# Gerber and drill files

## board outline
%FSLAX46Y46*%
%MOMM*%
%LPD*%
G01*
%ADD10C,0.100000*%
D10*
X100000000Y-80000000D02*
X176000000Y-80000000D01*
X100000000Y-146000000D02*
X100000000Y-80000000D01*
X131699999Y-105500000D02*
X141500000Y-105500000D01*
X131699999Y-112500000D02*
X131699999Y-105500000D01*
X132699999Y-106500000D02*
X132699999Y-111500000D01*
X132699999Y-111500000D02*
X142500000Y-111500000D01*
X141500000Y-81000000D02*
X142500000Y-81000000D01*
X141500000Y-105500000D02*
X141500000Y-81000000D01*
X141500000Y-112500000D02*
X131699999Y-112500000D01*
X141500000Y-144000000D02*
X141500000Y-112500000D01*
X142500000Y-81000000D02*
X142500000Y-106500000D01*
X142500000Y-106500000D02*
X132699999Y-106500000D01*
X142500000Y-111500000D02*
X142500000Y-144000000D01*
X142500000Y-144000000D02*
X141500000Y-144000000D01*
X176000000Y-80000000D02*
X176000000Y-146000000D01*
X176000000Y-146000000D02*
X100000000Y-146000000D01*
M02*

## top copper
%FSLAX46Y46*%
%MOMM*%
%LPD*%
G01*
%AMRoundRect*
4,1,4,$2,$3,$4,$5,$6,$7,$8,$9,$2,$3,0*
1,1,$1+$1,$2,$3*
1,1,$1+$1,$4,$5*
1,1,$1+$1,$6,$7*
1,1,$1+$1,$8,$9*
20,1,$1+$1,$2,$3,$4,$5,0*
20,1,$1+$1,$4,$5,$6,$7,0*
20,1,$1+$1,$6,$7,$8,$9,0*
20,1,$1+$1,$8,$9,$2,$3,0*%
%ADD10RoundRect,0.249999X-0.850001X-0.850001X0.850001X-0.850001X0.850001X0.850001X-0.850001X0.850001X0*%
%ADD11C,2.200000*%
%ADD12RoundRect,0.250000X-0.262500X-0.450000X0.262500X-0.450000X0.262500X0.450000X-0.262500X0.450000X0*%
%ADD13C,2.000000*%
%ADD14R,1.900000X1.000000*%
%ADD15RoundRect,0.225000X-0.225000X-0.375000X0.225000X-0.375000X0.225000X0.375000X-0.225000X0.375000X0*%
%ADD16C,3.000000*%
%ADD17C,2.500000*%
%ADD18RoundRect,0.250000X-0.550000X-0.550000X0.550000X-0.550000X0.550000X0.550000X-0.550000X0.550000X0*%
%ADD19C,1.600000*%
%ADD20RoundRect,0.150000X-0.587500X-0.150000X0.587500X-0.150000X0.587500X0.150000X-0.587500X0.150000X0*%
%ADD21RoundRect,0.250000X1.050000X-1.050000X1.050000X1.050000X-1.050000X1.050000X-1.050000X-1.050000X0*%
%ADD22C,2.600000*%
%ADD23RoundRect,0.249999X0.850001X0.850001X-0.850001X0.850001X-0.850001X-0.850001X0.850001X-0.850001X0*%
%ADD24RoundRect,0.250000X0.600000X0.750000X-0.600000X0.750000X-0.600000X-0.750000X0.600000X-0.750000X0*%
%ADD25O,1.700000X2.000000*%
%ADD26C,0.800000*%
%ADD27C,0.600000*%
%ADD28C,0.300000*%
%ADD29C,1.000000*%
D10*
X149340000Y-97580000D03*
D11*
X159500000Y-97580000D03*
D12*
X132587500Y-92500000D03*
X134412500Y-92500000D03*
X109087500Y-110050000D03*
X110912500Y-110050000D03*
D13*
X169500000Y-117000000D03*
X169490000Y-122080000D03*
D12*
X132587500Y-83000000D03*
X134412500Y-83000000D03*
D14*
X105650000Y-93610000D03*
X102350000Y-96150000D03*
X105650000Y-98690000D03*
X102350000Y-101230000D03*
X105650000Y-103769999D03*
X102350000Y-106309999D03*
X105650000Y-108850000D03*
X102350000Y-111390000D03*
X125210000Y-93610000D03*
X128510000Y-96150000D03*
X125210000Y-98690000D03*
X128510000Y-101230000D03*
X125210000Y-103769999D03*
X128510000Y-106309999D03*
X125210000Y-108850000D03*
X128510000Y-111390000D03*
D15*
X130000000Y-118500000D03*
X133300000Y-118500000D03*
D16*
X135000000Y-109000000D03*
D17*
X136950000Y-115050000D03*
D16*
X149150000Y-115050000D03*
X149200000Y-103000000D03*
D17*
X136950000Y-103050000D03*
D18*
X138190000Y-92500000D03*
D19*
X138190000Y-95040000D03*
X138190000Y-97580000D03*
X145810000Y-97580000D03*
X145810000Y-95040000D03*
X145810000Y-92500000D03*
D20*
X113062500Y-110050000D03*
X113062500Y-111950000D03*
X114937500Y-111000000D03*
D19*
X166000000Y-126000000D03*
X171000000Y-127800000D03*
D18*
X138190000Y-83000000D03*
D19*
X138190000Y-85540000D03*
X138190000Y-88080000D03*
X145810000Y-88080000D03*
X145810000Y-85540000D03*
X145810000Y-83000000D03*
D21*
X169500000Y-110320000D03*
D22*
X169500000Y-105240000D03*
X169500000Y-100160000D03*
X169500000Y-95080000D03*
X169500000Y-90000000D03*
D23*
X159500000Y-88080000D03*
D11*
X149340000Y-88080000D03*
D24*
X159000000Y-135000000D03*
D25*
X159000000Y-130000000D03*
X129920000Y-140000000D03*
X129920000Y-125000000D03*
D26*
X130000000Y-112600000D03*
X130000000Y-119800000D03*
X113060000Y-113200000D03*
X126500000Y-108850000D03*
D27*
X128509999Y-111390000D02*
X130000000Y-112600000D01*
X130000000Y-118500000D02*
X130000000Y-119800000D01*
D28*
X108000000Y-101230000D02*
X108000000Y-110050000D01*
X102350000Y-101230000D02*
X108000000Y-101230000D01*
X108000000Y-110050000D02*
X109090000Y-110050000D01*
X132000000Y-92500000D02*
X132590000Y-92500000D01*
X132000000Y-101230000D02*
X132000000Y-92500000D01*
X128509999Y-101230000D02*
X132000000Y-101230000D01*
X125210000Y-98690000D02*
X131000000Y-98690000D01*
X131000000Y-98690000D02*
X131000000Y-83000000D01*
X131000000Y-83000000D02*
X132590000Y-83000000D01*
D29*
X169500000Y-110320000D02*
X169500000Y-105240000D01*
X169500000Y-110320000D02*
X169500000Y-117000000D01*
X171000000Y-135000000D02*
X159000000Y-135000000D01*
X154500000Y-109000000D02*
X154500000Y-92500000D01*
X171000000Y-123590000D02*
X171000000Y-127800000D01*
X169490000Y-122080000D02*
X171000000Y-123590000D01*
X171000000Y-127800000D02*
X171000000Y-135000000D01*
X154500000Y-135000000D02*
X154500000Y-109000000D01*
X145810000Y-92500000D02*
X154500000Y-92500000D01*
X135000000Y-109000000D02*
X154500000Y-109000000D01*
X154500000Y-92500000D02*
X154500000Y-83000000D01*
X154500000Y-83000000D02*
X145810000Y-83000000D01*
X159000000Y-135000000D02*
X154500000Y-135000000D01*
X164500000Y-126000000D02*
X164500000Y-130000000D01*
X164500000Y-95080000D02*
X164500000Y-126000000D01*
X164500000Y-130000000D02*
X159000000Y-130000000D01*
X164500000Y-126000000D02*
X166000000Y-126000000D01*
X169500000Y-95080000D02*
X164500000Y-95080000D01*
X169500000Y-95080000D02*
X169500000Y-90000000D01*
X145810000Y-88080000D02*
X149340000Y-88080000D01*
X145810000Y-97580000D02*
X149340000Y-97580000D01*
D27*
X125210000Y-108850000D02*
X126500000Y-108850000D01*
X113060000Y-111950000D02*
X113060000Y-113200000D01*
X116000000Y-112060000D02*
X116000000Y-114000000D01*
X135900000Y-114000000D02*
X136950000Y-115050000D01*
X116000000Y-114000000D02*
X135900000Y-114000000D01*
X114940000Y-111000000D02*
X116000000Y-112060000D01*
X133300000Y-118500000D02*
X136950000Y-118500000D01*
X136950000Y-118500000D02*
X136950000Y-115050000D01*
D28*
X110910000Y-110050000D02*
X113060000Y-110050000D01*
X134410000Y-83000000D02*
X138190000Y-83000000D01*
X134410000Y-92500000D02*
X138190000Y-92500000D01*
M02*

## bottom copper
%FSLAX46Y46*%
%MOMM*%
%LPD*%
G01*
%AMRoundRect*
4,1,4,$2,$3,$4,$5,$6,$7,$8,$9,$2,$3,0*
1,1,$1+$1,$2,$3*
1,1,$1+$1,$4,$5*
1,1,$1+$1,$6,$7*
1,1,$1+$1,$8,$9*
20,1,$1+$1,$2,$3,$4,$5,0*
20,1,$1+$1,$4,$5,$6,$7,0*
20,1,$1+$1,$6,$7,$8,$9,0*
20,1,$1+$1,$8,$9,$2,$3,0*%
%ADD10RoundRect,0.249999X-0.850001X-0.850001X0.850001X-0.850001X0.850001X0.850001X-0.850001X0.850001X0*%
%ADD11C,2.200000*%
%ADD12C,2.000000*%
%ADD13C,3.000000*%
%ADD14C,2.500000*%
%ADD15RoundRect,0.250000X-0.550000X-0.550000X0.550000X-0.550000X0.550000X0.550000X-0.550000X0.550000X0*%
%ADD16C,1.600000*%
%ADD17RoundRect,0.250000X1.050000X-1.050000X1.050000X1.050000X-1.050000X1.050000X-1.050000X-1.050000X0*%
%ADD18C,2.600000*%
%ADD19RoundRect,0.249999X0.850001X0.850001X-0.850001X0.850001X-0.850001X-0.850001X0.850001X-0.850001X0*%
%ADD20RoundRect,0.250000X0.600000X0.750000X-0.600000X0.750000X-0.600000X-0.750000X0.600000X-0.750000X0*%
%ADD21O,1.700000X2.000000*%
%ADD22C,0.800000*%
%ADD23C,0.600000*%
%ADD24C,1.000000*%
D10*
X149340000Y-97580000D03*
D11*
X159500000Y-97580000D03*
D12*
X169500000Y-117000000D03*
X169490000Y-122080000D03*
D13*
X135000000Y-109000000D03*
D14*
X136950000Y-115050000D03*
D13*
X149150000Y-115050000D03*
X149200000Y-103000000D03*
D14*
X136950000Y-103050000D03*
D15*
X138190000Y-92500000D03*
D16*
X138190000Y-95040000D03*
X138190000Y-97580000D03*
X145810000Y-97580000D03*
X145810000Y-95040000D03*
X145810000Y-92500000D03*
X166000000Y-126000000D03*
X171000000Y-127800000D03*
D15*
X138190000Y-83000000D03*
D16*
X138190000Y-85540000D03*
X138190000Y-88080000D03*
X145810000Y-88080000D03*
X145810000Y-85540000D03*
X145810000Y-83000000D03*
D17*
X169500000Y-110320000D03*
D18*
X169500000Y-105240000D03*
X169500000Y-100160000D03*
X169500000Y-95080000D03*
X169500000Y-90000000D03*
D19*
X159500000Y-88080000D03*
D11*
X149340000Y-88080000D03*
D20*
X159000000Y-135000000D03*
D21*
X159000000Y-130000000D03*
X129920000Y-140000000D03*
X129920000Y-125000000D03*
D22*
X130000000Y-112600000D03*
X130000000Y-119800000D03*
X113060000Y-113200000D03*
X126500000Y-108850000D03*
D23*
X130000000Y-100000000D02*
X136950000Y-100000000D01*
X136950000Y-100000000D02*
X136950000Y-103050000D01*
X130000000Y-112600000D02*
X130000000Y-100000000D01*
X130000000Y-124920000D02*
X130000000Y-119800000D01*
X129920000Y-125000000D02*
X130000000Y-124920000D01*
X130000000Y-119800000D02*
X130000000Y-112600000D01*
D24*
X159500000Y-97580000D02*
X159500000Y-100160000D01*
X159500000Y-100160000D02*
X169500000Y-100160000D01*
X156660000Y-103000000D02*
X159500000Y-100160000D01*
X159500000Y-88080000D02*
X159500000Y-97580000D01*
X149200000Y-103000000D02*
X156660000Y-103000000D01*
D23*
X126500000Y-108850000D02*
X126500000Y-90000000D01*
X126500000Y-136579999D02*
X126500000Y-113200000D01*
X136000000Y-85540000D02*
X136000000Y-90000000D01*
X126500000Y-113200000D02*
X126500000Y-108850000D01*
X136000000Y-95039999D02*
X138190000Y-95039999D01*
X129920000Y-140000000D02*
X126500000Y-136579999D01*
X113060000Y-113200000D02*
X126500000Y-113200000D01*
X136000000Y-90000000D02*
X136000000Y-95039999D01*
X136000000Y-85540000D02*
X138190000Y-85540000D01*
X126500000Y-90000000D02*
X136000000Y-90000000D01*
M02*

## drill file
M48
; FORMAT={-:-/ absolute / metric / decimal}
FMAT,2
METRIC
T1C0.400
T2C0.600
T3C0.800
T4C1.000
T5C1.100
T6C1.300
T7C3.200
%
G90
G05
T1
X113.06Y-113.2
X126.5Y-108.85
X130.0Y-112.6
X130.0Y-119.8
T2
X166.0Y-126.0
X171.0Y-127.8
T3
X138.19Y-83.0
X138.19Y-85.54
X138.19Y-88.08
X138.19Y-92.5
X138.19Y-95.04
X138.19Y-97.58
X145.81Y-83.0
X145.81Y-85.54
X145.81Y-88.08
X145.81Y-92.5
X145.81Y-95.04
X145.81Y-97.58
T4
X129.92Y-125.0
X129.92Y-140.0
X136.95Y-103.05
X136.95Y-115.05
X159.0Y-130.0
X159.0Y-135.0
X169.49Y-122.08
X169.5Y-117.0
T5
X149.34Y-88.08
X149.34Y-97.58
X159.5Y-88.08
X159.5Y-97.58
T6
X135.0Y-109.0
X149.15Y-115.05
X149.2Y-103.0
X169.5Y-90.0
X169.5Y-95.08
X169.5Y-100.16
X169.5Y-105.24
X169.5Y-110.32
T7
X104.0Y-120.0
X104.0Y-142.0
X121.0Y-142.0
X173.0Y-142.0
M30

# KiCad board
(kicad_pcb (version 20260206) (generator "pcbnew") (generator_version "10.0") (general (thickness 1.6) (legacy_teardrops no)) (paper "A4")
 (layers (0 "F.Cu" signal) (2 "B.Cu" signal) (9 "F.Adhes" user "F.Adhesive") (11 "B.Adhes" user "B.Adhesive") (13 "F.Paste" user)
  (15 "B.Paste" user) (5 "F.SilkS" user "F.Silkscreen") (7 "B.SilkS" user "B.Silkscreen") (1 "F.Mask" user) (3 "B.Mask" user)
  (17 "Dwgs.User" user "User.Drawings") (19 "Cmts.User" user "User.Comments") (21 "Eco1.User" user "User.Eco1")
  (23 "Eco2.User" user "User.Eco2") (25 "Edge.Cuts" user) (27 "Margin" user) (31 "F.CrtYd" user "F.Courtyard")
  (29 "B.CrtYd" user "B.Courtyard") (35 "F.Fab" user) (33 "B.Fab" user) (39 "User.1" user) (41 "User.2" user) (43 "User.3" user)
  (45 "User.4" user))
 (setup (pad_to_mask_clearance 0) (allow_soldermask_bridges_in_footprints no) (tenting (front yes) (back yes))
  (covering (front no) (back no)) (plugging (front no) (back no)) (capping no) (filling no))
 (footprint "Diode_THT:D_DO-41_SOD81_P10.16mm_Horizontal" (layer "F.Cu") (at 149.34 97.58)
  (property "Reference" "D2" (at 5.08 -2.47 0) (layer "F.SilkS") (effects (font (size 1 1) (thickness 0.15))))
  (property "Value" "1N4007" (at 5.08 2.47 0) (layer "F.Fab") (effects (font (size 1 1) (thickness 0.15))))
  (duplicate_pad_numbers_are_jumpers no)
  (pad "1" thru_hole roundrect (at 0 0) (size 2.2 2.2) (drill 1.1) (layers "*.Cu" "*.Mask") (remove_unused_layers no)
   (roundrect_rratio 0.113636) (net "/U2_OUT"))
  (pad "2" thru_hole circle (at 10.16 0) (size 2.2 2.2) (drill 1.1) (layers "*.Cu" "*.Mask") (remove_unused_layers no) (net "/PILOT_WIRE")))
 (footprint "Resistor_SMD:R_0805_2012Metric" (layer "F.Cu") (at 133.5 92.5)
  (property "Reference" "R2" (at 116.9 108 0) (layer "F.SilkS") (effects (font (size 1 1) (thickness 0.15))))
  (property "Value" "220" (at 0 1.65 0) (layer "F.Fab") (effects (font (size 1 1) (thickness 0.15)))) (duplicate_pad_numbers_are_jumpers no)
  (pad "1" smd roundrect (at -0.9125 0) (size 1.025 1.4) (layers "F.Cu" "F.Mask" "F.Paste") (roundrect_rratio 0.243902) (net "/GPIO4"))
  (pad "2" smd roundrect (at 0.9125 0) (size 1.025 1.4) (layers "F.Cu" "F.Mask" "F.Paste") (roundrect_rratio 0.243902) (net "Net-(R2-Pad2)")))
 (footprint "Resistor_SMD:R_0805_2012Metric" (layer "F.Cu") (at 110 110.05)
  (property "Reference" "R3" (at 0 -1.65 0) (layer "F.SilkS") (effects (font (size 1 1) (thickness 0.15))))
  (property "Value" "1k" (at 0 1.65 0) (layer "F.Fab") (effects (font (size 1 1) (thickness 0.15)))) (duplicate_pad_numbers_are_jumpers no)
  (pad "1" smd roundrect (at -0.9125 0) (size 1.025 1.4) (layers "F.Cu" "F.Mask" "F.Paste") (roundrect_rratio 0.243902) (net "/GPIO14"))
  (pad "2" smd roundrect (at 0.9125 0) (size 1.025 1.4) (layers "F.Cu" "F.Mask" "F.Paste") (roundrect_rratio 0.243902) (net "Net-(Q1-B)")))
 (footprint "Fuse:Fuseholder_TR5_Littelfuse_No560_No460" (layer "F.Cu") (at 169.5 117 -90)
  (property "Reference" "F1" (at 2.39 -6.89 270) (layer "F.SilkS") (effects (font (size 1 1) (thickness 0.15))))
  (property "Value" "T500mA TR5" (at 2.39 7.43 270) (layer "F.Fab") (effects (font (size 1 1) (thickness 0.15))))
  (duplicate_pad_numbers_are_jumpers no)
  (pad "1" thru_hole circle (at 0 0 270) (size 2 2) (drill 1) (layers "*.Cu" "*.Mask") (remove_unused_layers no) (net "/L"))
  (pad "2" thru_hole circle (at 5.08 0.01 270) (size 2 2) (drill 1) (layers "*.Cu" "*.Mask") (remove_unused_layers no) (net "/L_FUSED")))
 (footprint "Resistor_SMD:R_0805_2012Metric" (layer "F.Cu") (at 133.5 83)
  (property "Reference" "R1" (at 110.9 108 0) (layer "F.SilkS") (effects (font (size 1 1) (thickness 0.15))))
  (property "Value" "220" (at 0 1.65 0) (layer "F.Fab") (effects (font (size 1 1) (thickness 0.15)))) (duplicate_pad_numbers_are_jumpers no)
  (pad "1" smd roundrect (at -0.9125 0) (size 1.025 1.4) (layers "F.Cu" "F.Mask" "F.Paste") (roundrect_rratio 0.243902) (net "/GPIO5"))
  (pad "2" smd roundrect (at 0.9125 0) (size 1.025 1.4) (layers "F.Cu" "F.Mask" "F.Paste") (roundrect_rratio 0.243902) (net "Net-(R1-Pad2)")))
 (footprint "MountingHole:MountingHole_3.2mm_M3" (layer "F.Cu") (at 121 142)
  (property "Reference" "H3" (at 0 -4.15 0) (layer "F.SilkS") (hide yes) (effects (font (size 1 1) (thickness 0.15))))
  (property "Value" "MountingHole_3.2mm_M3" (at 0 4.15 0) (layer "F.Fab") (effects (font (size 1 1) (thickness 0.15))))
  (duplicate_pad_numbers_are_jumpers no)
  (pad "" np_thru_hole circle (at 0 0) (size 3.2 3.2) (drill 3.2) (layers "*.Cu" "*.Mask")))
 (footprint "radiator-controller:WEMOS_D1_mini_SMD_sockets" (layer "F.Cu") (at 115.43 102.5)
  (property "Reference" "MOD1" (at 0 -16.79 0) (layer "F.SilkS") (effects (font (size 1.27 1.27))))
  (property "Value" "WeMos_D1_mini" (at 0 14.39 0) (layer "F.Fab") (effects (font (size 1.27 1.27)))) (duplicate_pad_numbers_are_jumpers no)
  (pad "1" smd rect (at -9.78 -8.89) (size 1.9 1) (layers "F.Cu" "F.Mask" "F.Paste") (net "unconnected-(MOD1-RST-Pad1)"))
  (pad "2" smd rect (at -13.08 -6.35) (size 1.9 1) (layers "F.Cu" "F.Mask" "F.Paste") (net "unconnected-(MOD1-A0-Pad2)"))
  (pad "3" smd rect (at -9.78 -3.81) (size 1.9 1) (layers "F.Cu" "F.Mask" "F.Paste") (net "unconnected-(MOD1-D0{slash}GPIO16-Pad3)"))
  (pad "4" smd rect (at -13.08 -1.27) (size 1.9 1) (layers "F.Cu" "F.Mask" "F.Paste") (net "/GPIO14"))
  (pad "5" smd rect (at -9.78 1.269999) (size 1.9 1) (layers "F.Cu" "F.Mask" "F.Paste") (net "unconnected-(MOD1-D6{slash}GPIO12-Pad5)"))
  (pad "6" smd rect (at -13.08 3.809999) (size 1.9 1) (layers "F.Cu" "F.Mask" "F.Paste") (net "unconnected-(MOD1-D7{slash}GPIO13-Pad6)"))
  (pad "7" smd rect (at -9.78 6.35) (size 1.9 1) (layers "F.Cu" "F.Mask" "F.Paste") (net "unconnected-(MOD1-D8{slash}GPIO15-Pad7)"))
  (pad "8" smd rect (at -13.08 8.89) (size 1.9 1) (layers "F.Cu" "F.Mask" "F.Paste") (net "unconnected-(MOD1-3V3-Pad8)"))
  (pad "9" smd rect (at 9.78 -8.89) (size 1.9 1) (layers "F.Cu" "F.Mask" "F.Paste") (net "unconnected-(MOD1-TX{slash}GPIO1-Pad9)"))
  (pad "10" smd rect (at 13.08 -6.35) (size 1.9 1) (layers "F.Cu" "F.Mask" "F.Paste") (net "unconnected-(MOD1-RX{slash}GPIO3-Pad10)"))
  (pad "11" smd rect (at 9.78 -3.81) (size 1.9 1) (layers "F.Cu" "F.Mask" "F.Paste") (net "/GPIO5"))
  (pad "12" smd rect (at 13.08 -1.27) (size 1.9 1) (layers "F.Cu" "F.Mask" "F.Paste") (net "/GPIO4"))
  (pad "13" smd rect (at 9.78 1.269999) (size 1.9 1) (layers "F.Cu" "F.Mask" "F.Paste") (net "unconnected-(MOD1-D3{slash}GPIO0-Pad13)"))
  (pad "14" smd rect (at 13.08 3.809999) (size 1.9 1) (layers "F.Cu" "F.Mask" "F.Paste") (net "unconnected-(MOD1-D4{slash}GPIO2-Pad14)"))
  (pad "15" smd rect (at 9.78 6.35) (size 1.9 1) (layers "F.Cu" "F.Mask" "F.Paste") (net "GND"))
  (pad "16" smd rect (at 13.08 8.89) (size 1.9 1) (layers "F.Cu" "F.Mask" "F.Paste") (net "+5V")))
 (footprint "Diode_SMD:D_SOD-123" (layer "F.Cu") (at 131.65 118.5)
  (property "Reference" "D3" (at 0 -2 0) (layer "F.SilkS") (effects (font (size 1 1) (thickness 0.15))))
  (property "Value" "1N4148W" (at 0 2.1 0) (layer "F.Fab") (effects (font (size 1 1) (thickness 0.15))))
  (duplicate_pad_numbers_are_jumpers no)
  (pad "1" smd roundrect (at -1.65 0) (size 0.9 1.2) (layers "F.Cu" "F.Mask" "F.Paste") (roundrect_rratio 0.25) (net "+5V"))
  (pad "2" smd roundrect (at 1.65 0) (size 0.9 1.2) (layers "F.Cu" "F.Mask" "F.Paste") (roundrect_rratio 0.25) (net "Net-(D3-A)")))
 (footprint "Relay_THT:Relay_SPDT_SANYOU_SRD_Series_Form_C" (layer "F.Cu") (at 135 109)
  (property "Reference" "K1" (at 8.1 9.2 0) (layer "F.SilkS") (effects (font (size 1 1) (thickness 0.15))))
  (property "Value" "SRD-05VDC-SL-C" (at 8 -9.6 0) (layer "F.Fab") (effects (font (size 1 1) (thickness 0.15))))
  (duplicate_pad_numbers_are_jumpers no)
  (pad "1" thru_hole circle (at 0 0 90) (size 3 3) (drill 1.3) (layers "*.Cu" "*.Mask") (remove_unused_layers no) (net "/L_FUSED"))
  (pad "2" thru_hole circle (at 1.95 6.05 90) (size 2.5 2.5) (drill 1) (layers "*.Cu" "*.Mask") (remove_unused_layers no) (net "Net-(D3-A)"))
  (pad "3" thru_hole circle (at 14.15 6.05 90) (size 3 3) (drill 1.3) (layers "*.Cu" "*.Mask") (remove_unused_layers no)
   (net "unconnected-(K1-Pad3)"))
  (pad "4" thru_hole circle (at 14.2 -6 90) (size 3 3) (drill 1.3) (layers "*.Cu" "*.Mask") (remove_unused_layers no) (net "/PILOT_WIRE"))
  (pad "5" thru_hole circle (at 1.95 -5.95 90) (size 2.5 2.5) (drill 1) (layers "*.Cu" "*.Mask") (remove_unused_layers no) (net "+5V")))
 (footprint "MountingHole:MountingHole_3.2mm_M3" (layer "F.Cu") (at 104 142)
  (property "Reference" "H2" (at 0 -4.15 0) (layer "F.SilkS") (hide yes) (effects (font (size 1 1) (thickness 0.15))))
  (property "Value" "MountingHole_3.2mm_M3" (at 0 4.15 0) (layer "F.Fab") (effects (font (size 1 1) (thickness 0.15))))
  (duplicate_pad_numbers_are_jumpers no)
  (pad "" np_thru_hole circle (at 0 0) (size 3.2 3.2) (drill 3.2) (layers "*.Cu" "*.Mask")))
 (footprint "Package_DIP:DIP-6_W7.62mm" (layer "F.Cu") (at 138.19 92.5)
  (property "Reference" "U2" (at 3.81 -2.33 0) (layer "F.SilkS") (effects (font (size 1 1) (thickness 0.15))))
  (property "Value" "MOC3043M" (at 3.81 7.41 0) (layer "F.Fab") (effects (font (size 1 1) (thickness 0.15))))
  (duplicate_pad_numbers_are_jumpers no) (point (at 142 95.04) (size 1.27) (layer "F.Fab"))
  (pad "1" thru_hole roundrect (at 0 0) (size 1.6 1.6) (drill 0.8) (layers "*.Cu" "*.Mask") (remove_unused_layers no)
   (roundrect_rratio 0.15625) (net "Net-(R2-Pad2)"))
  (pad "2" thru_hole circle (at 0 2.54) (size 1.6 1.6) (drill 0.8) (layers "*.Cu" "*.Mask") (remove_unused_layers no) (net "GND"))
  (pad "3" thru_hole circle (at 0 5.08) (size 1.6 1.6) (drill 0.8) (layers "*.Cu" "*.Mask") (remove_unused_layers no)
   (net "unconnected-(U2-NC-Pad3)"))
  (pad "4" thru_hole circle (at 7.62 5.08) (size 1.6 1.6) (drill 0.8) (layers "*.Cu" "*.Mask") (remove_unused_layers no) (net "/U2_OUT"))
  (pad "5" thru_hole circle (at 7.62 2.54) (size 1.6 1.6) (drill 0.8) (layers "*.Cu" "*.Mask") (remove_unused_layers no)
   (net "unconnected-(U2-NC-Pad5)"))
  (pad "6" thru_hole circle (at 7.62 0) (size 1.6 1.6) (drill 0.8) (layers "*.Cu" "*.Mask") (remove_unused_layers no) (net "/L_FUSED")))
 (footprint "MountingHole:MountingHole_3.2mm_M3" (layer "F.Cu") (at 173 142)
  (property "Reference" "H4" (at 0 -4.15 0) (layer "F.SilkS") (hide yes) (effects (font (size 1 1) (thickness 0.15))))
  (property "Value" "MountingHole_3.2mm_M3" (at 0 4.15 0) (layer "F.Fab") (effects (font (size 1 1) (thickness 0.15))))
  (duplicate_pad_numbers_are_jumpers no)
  (pad "" np_thru_hole circle (at 0 0) (size 3.2 3.2) (drill 3.2) (layers "*.Cu" "*.Mask")))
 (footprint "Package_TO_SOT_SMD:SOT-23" (layer "F.Cu") (at 114 111)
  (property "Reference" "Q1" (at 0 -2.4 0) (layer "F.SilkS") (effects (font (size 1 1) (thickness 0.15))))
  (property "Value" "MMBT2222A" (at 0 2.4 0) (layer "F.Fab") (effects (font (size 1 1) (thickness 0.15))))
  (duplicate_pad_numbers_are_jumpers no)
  (pad "1" smd roundrect (at -0.9375 -0.95) (size 1.475 0.6) (layers "F.Cu" "F.Mask" "F.Paste") (roundrect_rratio 0.25) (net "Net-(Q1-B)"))
  (pad "2" smd roundrect (at -0.9375 0.95) (size 1.475 0.6) (layers "F.Cu" "F.Mask" "F.Paste") (roundrect_rratio 0.25) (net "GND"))
  (pad "3" smd roundrect (at 0.9375 0) (size 1.475 0.6) (layers "F.Cu" "F.Mask" "F.Paste") (roundrect_rratio 0.25) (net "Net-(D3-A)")))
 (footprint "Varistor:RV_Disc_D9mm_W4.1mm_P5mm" (layer "F.Cu") (at 166 126)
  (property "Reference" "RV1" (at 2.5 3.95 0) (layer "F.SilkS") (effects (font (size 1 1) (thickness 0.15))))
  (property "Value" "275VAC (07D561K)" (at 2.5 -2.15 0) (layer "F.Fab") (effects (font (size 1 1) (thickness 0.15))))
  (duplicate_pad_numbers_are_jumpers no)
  (pad "1" thru_hole circle (at 0 0) (size 1.6 1.6) (drill 0.6) (layers "*.Cu" "*.Mask") (remove_unused_layers no) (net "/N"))
  (pad "2" thru_hole circle (at 5 1.8) (size 1.6 1.6) (drill 0.6) (layers "*.Cu" "*.Mask") (remove_unused_layers no) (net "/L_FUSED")))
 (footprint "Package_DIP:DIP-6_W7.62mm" (layer "F.Cu") (at 138.19 83)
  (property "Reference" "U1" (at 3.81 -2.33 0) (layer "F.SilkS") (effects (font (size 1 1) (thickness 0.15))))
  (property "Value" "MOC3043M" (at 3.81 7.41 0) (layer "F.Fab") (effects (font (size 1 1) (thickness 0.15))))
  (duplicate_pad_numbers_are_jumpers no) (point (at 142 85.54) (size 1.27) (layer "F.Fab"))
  (pad "1" thru_hole roundrect (at 0 0) (size 1.6 1.6) (drill 0.8) (layers "*.Cu" "*.Mask") (remove_unused_layers no)
   (roundrect_rratio 0.15625) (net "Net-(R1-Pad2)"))
  (pad "2" thru_hole circle (at 0 2.54) (size 1.6 1.6) (drill 0.8) (layers "*.Cu" "*.Mask") (remove_unused_layers no) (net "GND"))
  (pad "3" thru_hole circle (at 0 5.08) (size 1.6 1.6) (drill 0.8) (layers "*.Cu" "*.Mask") (remove_unused_layers no)
   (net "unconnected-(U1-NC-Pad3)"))
  (pad "4" thru_hole circle (at 7.62 5.08) (size 1.6 1.6) (drill 0.8) (layers "*.Cu" "*.Mask") (remove_unused_layers no) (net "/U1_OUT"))
  (pad "5" thru_hole circle (at 7.62 2.54) (size 1.6 1.6) (drill 0.8) (layers "*.Cu" "*.Mask") (remove_unused_layers no)
   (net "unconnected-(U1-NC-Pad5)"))
  (pad "6" thru_hole circle (at 7.62 0) (size 1.6 1.6) (drill 0.8) (layers "*.Cu" "*.Mask") (remove_unused_layers no) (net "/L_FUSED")))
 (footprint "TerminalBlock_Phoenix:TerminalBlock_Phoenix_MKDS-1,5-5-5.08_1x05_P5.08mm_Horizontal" (layer "F.Cu") (at 169.5 110.32 90)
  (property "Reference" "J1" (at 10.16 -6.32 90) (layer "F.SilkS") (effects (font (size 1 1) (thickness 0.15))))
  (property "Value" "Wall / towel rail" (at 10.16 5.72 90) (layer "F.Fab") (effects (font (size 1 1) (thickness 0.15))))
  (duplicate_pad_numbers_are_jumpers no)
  (pad "1" thru_hole roundrect (at 0 0 90) (size 2.6 2.6) (drill 1.3) (layers "*.Cu" "*.Mask") (remove_unused_layers no)
   (roundrect_rratio 0.096154) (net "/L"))
  (pad "2" thru_hole circle (at 5.08 0 90) (size 2.6 2.6) (drill 1.3) (layers "*.Cu" "*.Mask") (remove_unused_layers no) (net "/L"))
  (pad "3" thru_hole circle (at 10.16 0 90) (size 2.6 2.6) (drill 1.3) (layers "*.Cu" "*.Mask") (remove_unused_layers no)
   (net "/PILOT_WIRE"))
  (pad "4" thru_hole circle (at 15.24 0 90) (size 2.6 2.6) (drill 1.3) (layers "*.Cu" "*.Mask") (remove_unused_layers no) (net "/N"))
  (pad "5" thru_hole circle (at 20.32 0 90) (size 2.6 2.6) (drill 1.3) (layers "*.Cu" "*.Mask") (remove_unused_layers no) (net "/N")))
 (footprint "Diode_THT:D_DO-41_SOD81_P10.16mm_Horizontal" (layer "F.Cu") (at 159.5 88.08 180)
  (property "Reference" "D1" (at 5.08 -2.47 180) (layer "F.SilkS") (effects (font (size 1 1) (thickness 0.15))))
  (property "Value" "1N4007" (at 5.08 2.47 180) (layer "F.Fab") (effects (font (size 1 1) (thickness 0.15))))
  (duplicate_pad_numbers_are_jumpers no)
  (pad "1" thru_hole roundrect (at 0 0 180) (size 2.2 2.2) (drill 1.1) (layers "*.Cu" "*.Mask") (remove_unused_layers no)
   (roundrect_rratio 0.113636) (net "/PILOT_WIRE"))
  (pad "2" thru_hole circle (at 10.16 0 180) (size 2.2 2.2) (drill 1.1) (layers "*.Cu" "*.Mask") (remove_unused_layers no) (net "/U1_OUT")))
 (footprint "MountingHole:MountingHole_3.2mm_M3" (layer "F.Cu") (at 104 120)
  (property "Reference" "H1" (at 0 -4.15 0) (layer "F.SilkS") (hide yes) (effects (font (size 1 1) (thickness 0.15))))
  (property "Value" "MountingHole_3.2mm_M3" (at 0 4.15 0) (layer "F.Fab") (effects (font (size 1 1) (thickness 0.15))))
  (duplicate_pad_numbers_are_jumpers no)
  (pad "" np_thru_hole circle (at 0 0) (size 3.2 3.2) (drill 3.2) (layers "*.Cu" "*.Mask")))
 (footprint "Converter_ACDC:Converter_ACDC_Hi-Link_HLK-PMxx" (layer "F.Cu") (at 159 135 180)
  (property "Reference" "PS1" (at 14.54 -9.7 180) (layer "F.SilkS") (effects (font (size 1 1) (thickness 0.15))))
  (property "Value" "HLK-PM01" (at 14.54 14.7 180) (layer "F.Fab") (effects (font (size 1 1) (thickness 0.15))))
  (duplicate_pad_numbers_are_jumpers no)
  (pad "1" thru_hole roundrect (at 0 0 180) (size 1.7 2) (drill 1) (layers "*.Cu" "*.Mask") (remove_unused_layers no)
   (roundrect_rratio 0.147059) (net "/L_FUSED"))
  (pad "2" thru_hole oval (at 0 5 180) (size 1.7 2) (drill 1) (layers "*.Cu" "*.Mask") (remove_unused_layers no) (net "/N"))
  (pad "3" thru_hole oval (at 29.08 -5 180) (size 1.7 2) (drill 1) (layers "*.Cu" "*.Mask") (remove_unused_layers no) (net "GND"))
  (pad "4" thru_hole oval (at 29.08 10 180) (size 1.7 2) (drill 1) (layers "*.Cu" "*.Mask") (remove_unused_layers no) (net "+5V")))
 (gr_line (start 100 80) (end 176 80) (stroke (width 0.1) (type default)) (layer "Edge.Cuts"))
 (gr_line (start 100 146) (end 100 80) (stroke (width 0.1) (type default)) (layer "Edge.Cuts"))
 (gr_line (start 131.699999 105.5) (end 141.5 105.5) (stroke (width 0.1) (type default)) (layer "Edge.Cuts"))
 (gr_line (start 131.699999 112.5) (end 131.699999 105.5) (stroke (width 0.1) (type default)) (layer "Edge.Cuts"))
 (gr_line (start 132.699999 106.5) (end 132.699999 111.5) (stroke (width 0.1) (type default)) (layer "Edge.Cuts"))
 (gr_line (start 132.699999 111.5) (end 142.5 111.5) (stroke (width 0.1) (type default)) (layer "Edge.Cuts"))
 (gr_line (start 141.5 81) (end 142.5 81) (stroke (width 0.1) (type default)) (layer "Edge.Cuts"))
 (gr_line (start 141.5 105.5) (end 141.5 81) (stroke (width 0.1) (type default)) (layer "Edge.Cuts"))
 (gr_line (start 141.5 112.5) (end 131.699999 112.5) (stroke (width 0.1) (type default)) (layer "Edge.Cuts"))
 (gr_line (start 141.5 144) (end 141.5 112.5) (stroke (width 0.1) (type default)) (layer "Edge.Cuts"))
 (gr_line (start 142.5 81) (end 142.5 106.5) (stroke (width 0.1) (type default)) (layer "Edge.Cuts"))
 (gr_line (start 142.5 106.5) (end 132.699999 106.5) (stroke (width 0.1) (type default)) (layer "Edge.Cuts"))
 (gr_line (start 142.5 111.5) (end 142.5 144) (stroke (width 0.1) (type default)) (layer "Edge.Cuts"))
 (gr_line (start 142.5 144) (end 141.5 144) (stroke (width 0.1) (type default)) (layer "Edge.Cuts"))
 (gr_line (start 176 80) (end 176 146) (stroke (width 0.1) (type default)) (layer "Edge.Cuts"))
 (gr_line (start 176 146) (end 100 146) (stroke (width 0.1) (type default)) (layer "Edge.Cuts"))
 (segment (start 128.509999 111.39) (end 130 112.6) (width 0.6) (layer "F.Cu") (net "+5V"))
 (segment (start 130 118.5) (end 130 119.8) (width 0.6) (layer "F.Cu") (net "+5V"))
 (via (at 130 112.6) (size 0.8) (drill 0.4) (layers "F.Cu" "B.Cu") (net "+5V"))
 (via (at 130 119.8) (size 0.8) (drill 0.4) (layers "F.Cu" "B.Cu") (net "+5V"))
 (segment (start 130 100) (end 136.95 100) (width 0.6) (layer "B.Cu") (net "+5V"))
 (segment (start 136.95 100) (end 136.95 103.05) (width 0.6) (layer "B.Cu") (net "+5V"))
 (segment (start 130 112.6) (end 130 100) (width 0.6) (layer "B.Cu") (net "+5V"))
 (segment (start 130 124.92) (end 130 119.8) (width 0.6) (layer "B.Cu") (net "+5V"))
 (segment (start 129.92 125) (end 130 124.92) (width 0.6) (layer "B.Cu") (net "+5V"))
 (segment (start 130 119.8) (end 130 112.6) (width 0.6) (layer "B.Cu") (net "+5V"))
 (segment (start 108 101.23) (end 108 110.05) (width 0.3) (layer "F.Cu") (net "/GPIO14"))
 (segment (start 102.35 101.23) (end 108 101.23) (width 0.3) (layer "F.Cu") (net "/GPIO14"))
 (segment (start 108 110.05) (end 109.09 110.05) (width 0.3) (layer "F.Cu") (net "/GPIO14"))
 (segment (start 132 92.5) (end 132.59 92.5) (width 0.3) (layer "F.Cu") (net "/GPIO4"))
 (segment (start 132 101.23) (end 132 92.5) (width 0.3) (layer "F.Cu") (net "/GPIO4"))
 (segment (start 128.509999 101.23) (end 132 101.23) (width 0.3) (layer "F.Cu") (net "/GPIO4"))
 (segment (start 125.21 98.69) (end 131 98.69) (width 0.3) (layer "F.Cu") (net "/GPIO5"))
 (segment (start 131 98.69) (end 131 83) (width 0.3) (layer "F.Cu") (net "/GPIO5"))
 (segment (start 131 83) (end 132.59 83) (width 0.3) (layer "F.Cu") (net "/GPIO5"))
 (segment (start 169.5 110.32) (end 169.5 105.24) (width 1) (layer "F.Cu") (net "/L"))
 (segment (start 169.5 110.32) (end 169.5 117) (width 1) (layer "F.Cu") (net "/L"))
 (segment (start 171 135) (end 159 135) (width 1) (layer "F.Cu") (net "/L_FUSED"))
 (segment (start 154.5 109) (end 154.5 92.5) (width 1) (layer "F.Cu") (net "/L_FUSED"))
 (segment (start 171 123.59) (end 171 127.8) (width 1) (layer "F.Cu") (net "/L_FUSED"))
 (segment (start 169.49 122.08) (end 171 123.59) (width 1) (layer "F.Cu") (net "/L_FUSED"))
 (segment (start 171 127.8) (end 171 135) (width 1) (layer "F.Cu") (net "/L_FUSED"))
 (segment (start 154.5 135) (end 154.5 109) (width 1) (layer "F.Cu") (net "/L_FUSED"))
 (segment (start 145.81 92.5) (end 154.5 92.5) (width 1) (layer "F.Cu") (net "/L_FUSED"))
 (segment (start 135 109) (end 154.5 109) (width 1) (layer "F.Cu") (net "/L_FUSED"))
 (segment (start 154.5 92.5) (end 154.5 83) (width 1) (layer "F.Cu") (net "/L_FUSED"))
 (segment (start 154.5 83) (end 145.81 83) (width 1) (layer "F.Cu") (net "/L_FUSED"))
 (segment (start 159 135) (end 154.5 135) (width 1) (layer "F.Cu") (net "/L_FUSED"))
 (segment (start 164.5 126) (end 164.5 130) (width 1) (layer "F.Cu") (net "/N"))
 (segment (start 164.5 95.08) (end 164.5 126) (width 1) (layer "F.Cu") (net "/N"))
 (segment (start 164.5 130) (end 159 130) (width 1) (layer "F.Cu") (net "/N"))
 (segment (start 164.5 126) (end 166 126) (width 1) (layer "F.Cu") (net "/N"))
 (segment (start 169.5 95.08) (end 164.5 95.08) (width 1) (layer "F.Cu") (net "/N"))
 (segment (start 169.5 95.08) (end 169.5 90) (width 1) (layer "F.Cu") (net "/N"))
 (segment (start 159.5 97.58) (end 159.5 100.16) (width 1) (layer "B.Cu") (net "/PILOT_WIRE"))
 (segment (start 159.5 100.16) (end 169.5 100.16) (width 1) (layer "B.Cu") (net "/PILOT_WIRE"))
 (segment (start 156.66 103) (end 159.5 100.16) (width 1) (layer "B.Cu") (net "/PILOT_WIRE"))
 (segment (start 159.5 88.08) (end 159.5 97.58) (width 1) (layer "B.Cu") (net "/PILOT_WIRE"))
 (segment (start 149.2 103) (end 156.66 103) (width 1) (layer "B.Cu") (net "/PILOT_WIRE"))
 (segment (start 145.81 88.08) (end 149.34 88.08) (width 1) (layer "F.Cu") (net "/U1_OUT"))
 (segment (start 145.81 97.58) (end 149.34 97.58) (width 1) (layer "F.Cu") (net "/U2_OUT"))
 (segment (start 125.21 108.85) (end 126.5 108.85) (width 0.6) (layer "F.Cu") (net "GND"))
 (segment (start 113.06 111.95) (end 113.06 113.2) (width 0.6) (layer "F.Cu") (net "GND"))
 (via (at 113.06 113.2) (size 0.8) (drill 0.4) (layers "F.Cu" "B.Cu") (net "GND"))
 (via (at 126.5 108.85) (size 0.8) (drill 0.4) (layers "F.Cu" "B.Cu") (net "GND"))
 (segment (start 126.5 108.85) (end 126.5 90) (width 0.6) (layer "B.Cu") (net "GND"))
 (segment (start 126.5 136.579999) (end 126.5 113.2) (width 0.6) (layer "B.Cu") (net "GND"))
 (segment (start 136 85.54) (end 136 90) (width 0.6) (layer "B.Cu") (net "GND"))
 (segment (start 126.5 113.2) (end 126.5 108.85) (width 0.6) (layer "B.Cu") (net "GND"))
 (segment (start 136 95.039999) (end 138.19 95.039999) (width 0.6) (layer "B.Cu") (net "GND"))
 (segment (start 129.92 140) (end 126.5 136.579999) (width 0.6) (layer "B.Cu") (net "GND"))
 (segment (start 113.06 113.2) (end 126.5 113.2) (width 0.6) (layer "B.Cu") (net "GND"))
 (segment (start 136 90) (end 136 95.039999) (width 0.6) (layer "B.Cu") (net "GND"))
 (segment (start 136 85.54) (end 138.19 85.54) (width 0.6) (layer "B.Cu") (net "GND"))
 (segment (start 126.5 90) (end 136 90) (width 0.6) (layer "B.Cu") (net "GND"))
 (segment (start 116 112.06) (end 116 114) (width 0.6) (layer "F.Cu") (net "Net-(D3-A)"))
 (segment (start 135.9 114) (end 136.95 115.05) (width 0.6) (layer "F.Cu") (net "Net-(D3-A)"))
 (segment (start 116 114) (end 135.9 114) (width 0.6) (layer "F.Cu") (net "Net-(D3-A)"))
 (segment (start 114.94 111) (end 116 112.06) (width 0.6) (layer "F.Cu") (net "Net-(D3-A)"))
 (segment (start 133.3 118.5) (end 136.95 118.5) (width 0.6) (layer "F.Cu") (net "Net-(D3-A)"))
 (segment (start 136.95 118.5) (end 136.95 115.05) (width 0.6) (layer "F.Cu") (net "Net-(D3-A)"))
 (segment (start 110.91 110.05) (end 113.06 110.05) (width 0.3) (layer "F.Cu") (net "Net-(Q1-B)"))
 (segment (start 134.41 83) (end 138.19 83) (width 0.3) (layer "F.Cu") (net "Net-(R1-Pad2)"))
 (segment (start 134.41 92.5) (end 138.19 92.5) (width 0.3) (layer "F.Cu") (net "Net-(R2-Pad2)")))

